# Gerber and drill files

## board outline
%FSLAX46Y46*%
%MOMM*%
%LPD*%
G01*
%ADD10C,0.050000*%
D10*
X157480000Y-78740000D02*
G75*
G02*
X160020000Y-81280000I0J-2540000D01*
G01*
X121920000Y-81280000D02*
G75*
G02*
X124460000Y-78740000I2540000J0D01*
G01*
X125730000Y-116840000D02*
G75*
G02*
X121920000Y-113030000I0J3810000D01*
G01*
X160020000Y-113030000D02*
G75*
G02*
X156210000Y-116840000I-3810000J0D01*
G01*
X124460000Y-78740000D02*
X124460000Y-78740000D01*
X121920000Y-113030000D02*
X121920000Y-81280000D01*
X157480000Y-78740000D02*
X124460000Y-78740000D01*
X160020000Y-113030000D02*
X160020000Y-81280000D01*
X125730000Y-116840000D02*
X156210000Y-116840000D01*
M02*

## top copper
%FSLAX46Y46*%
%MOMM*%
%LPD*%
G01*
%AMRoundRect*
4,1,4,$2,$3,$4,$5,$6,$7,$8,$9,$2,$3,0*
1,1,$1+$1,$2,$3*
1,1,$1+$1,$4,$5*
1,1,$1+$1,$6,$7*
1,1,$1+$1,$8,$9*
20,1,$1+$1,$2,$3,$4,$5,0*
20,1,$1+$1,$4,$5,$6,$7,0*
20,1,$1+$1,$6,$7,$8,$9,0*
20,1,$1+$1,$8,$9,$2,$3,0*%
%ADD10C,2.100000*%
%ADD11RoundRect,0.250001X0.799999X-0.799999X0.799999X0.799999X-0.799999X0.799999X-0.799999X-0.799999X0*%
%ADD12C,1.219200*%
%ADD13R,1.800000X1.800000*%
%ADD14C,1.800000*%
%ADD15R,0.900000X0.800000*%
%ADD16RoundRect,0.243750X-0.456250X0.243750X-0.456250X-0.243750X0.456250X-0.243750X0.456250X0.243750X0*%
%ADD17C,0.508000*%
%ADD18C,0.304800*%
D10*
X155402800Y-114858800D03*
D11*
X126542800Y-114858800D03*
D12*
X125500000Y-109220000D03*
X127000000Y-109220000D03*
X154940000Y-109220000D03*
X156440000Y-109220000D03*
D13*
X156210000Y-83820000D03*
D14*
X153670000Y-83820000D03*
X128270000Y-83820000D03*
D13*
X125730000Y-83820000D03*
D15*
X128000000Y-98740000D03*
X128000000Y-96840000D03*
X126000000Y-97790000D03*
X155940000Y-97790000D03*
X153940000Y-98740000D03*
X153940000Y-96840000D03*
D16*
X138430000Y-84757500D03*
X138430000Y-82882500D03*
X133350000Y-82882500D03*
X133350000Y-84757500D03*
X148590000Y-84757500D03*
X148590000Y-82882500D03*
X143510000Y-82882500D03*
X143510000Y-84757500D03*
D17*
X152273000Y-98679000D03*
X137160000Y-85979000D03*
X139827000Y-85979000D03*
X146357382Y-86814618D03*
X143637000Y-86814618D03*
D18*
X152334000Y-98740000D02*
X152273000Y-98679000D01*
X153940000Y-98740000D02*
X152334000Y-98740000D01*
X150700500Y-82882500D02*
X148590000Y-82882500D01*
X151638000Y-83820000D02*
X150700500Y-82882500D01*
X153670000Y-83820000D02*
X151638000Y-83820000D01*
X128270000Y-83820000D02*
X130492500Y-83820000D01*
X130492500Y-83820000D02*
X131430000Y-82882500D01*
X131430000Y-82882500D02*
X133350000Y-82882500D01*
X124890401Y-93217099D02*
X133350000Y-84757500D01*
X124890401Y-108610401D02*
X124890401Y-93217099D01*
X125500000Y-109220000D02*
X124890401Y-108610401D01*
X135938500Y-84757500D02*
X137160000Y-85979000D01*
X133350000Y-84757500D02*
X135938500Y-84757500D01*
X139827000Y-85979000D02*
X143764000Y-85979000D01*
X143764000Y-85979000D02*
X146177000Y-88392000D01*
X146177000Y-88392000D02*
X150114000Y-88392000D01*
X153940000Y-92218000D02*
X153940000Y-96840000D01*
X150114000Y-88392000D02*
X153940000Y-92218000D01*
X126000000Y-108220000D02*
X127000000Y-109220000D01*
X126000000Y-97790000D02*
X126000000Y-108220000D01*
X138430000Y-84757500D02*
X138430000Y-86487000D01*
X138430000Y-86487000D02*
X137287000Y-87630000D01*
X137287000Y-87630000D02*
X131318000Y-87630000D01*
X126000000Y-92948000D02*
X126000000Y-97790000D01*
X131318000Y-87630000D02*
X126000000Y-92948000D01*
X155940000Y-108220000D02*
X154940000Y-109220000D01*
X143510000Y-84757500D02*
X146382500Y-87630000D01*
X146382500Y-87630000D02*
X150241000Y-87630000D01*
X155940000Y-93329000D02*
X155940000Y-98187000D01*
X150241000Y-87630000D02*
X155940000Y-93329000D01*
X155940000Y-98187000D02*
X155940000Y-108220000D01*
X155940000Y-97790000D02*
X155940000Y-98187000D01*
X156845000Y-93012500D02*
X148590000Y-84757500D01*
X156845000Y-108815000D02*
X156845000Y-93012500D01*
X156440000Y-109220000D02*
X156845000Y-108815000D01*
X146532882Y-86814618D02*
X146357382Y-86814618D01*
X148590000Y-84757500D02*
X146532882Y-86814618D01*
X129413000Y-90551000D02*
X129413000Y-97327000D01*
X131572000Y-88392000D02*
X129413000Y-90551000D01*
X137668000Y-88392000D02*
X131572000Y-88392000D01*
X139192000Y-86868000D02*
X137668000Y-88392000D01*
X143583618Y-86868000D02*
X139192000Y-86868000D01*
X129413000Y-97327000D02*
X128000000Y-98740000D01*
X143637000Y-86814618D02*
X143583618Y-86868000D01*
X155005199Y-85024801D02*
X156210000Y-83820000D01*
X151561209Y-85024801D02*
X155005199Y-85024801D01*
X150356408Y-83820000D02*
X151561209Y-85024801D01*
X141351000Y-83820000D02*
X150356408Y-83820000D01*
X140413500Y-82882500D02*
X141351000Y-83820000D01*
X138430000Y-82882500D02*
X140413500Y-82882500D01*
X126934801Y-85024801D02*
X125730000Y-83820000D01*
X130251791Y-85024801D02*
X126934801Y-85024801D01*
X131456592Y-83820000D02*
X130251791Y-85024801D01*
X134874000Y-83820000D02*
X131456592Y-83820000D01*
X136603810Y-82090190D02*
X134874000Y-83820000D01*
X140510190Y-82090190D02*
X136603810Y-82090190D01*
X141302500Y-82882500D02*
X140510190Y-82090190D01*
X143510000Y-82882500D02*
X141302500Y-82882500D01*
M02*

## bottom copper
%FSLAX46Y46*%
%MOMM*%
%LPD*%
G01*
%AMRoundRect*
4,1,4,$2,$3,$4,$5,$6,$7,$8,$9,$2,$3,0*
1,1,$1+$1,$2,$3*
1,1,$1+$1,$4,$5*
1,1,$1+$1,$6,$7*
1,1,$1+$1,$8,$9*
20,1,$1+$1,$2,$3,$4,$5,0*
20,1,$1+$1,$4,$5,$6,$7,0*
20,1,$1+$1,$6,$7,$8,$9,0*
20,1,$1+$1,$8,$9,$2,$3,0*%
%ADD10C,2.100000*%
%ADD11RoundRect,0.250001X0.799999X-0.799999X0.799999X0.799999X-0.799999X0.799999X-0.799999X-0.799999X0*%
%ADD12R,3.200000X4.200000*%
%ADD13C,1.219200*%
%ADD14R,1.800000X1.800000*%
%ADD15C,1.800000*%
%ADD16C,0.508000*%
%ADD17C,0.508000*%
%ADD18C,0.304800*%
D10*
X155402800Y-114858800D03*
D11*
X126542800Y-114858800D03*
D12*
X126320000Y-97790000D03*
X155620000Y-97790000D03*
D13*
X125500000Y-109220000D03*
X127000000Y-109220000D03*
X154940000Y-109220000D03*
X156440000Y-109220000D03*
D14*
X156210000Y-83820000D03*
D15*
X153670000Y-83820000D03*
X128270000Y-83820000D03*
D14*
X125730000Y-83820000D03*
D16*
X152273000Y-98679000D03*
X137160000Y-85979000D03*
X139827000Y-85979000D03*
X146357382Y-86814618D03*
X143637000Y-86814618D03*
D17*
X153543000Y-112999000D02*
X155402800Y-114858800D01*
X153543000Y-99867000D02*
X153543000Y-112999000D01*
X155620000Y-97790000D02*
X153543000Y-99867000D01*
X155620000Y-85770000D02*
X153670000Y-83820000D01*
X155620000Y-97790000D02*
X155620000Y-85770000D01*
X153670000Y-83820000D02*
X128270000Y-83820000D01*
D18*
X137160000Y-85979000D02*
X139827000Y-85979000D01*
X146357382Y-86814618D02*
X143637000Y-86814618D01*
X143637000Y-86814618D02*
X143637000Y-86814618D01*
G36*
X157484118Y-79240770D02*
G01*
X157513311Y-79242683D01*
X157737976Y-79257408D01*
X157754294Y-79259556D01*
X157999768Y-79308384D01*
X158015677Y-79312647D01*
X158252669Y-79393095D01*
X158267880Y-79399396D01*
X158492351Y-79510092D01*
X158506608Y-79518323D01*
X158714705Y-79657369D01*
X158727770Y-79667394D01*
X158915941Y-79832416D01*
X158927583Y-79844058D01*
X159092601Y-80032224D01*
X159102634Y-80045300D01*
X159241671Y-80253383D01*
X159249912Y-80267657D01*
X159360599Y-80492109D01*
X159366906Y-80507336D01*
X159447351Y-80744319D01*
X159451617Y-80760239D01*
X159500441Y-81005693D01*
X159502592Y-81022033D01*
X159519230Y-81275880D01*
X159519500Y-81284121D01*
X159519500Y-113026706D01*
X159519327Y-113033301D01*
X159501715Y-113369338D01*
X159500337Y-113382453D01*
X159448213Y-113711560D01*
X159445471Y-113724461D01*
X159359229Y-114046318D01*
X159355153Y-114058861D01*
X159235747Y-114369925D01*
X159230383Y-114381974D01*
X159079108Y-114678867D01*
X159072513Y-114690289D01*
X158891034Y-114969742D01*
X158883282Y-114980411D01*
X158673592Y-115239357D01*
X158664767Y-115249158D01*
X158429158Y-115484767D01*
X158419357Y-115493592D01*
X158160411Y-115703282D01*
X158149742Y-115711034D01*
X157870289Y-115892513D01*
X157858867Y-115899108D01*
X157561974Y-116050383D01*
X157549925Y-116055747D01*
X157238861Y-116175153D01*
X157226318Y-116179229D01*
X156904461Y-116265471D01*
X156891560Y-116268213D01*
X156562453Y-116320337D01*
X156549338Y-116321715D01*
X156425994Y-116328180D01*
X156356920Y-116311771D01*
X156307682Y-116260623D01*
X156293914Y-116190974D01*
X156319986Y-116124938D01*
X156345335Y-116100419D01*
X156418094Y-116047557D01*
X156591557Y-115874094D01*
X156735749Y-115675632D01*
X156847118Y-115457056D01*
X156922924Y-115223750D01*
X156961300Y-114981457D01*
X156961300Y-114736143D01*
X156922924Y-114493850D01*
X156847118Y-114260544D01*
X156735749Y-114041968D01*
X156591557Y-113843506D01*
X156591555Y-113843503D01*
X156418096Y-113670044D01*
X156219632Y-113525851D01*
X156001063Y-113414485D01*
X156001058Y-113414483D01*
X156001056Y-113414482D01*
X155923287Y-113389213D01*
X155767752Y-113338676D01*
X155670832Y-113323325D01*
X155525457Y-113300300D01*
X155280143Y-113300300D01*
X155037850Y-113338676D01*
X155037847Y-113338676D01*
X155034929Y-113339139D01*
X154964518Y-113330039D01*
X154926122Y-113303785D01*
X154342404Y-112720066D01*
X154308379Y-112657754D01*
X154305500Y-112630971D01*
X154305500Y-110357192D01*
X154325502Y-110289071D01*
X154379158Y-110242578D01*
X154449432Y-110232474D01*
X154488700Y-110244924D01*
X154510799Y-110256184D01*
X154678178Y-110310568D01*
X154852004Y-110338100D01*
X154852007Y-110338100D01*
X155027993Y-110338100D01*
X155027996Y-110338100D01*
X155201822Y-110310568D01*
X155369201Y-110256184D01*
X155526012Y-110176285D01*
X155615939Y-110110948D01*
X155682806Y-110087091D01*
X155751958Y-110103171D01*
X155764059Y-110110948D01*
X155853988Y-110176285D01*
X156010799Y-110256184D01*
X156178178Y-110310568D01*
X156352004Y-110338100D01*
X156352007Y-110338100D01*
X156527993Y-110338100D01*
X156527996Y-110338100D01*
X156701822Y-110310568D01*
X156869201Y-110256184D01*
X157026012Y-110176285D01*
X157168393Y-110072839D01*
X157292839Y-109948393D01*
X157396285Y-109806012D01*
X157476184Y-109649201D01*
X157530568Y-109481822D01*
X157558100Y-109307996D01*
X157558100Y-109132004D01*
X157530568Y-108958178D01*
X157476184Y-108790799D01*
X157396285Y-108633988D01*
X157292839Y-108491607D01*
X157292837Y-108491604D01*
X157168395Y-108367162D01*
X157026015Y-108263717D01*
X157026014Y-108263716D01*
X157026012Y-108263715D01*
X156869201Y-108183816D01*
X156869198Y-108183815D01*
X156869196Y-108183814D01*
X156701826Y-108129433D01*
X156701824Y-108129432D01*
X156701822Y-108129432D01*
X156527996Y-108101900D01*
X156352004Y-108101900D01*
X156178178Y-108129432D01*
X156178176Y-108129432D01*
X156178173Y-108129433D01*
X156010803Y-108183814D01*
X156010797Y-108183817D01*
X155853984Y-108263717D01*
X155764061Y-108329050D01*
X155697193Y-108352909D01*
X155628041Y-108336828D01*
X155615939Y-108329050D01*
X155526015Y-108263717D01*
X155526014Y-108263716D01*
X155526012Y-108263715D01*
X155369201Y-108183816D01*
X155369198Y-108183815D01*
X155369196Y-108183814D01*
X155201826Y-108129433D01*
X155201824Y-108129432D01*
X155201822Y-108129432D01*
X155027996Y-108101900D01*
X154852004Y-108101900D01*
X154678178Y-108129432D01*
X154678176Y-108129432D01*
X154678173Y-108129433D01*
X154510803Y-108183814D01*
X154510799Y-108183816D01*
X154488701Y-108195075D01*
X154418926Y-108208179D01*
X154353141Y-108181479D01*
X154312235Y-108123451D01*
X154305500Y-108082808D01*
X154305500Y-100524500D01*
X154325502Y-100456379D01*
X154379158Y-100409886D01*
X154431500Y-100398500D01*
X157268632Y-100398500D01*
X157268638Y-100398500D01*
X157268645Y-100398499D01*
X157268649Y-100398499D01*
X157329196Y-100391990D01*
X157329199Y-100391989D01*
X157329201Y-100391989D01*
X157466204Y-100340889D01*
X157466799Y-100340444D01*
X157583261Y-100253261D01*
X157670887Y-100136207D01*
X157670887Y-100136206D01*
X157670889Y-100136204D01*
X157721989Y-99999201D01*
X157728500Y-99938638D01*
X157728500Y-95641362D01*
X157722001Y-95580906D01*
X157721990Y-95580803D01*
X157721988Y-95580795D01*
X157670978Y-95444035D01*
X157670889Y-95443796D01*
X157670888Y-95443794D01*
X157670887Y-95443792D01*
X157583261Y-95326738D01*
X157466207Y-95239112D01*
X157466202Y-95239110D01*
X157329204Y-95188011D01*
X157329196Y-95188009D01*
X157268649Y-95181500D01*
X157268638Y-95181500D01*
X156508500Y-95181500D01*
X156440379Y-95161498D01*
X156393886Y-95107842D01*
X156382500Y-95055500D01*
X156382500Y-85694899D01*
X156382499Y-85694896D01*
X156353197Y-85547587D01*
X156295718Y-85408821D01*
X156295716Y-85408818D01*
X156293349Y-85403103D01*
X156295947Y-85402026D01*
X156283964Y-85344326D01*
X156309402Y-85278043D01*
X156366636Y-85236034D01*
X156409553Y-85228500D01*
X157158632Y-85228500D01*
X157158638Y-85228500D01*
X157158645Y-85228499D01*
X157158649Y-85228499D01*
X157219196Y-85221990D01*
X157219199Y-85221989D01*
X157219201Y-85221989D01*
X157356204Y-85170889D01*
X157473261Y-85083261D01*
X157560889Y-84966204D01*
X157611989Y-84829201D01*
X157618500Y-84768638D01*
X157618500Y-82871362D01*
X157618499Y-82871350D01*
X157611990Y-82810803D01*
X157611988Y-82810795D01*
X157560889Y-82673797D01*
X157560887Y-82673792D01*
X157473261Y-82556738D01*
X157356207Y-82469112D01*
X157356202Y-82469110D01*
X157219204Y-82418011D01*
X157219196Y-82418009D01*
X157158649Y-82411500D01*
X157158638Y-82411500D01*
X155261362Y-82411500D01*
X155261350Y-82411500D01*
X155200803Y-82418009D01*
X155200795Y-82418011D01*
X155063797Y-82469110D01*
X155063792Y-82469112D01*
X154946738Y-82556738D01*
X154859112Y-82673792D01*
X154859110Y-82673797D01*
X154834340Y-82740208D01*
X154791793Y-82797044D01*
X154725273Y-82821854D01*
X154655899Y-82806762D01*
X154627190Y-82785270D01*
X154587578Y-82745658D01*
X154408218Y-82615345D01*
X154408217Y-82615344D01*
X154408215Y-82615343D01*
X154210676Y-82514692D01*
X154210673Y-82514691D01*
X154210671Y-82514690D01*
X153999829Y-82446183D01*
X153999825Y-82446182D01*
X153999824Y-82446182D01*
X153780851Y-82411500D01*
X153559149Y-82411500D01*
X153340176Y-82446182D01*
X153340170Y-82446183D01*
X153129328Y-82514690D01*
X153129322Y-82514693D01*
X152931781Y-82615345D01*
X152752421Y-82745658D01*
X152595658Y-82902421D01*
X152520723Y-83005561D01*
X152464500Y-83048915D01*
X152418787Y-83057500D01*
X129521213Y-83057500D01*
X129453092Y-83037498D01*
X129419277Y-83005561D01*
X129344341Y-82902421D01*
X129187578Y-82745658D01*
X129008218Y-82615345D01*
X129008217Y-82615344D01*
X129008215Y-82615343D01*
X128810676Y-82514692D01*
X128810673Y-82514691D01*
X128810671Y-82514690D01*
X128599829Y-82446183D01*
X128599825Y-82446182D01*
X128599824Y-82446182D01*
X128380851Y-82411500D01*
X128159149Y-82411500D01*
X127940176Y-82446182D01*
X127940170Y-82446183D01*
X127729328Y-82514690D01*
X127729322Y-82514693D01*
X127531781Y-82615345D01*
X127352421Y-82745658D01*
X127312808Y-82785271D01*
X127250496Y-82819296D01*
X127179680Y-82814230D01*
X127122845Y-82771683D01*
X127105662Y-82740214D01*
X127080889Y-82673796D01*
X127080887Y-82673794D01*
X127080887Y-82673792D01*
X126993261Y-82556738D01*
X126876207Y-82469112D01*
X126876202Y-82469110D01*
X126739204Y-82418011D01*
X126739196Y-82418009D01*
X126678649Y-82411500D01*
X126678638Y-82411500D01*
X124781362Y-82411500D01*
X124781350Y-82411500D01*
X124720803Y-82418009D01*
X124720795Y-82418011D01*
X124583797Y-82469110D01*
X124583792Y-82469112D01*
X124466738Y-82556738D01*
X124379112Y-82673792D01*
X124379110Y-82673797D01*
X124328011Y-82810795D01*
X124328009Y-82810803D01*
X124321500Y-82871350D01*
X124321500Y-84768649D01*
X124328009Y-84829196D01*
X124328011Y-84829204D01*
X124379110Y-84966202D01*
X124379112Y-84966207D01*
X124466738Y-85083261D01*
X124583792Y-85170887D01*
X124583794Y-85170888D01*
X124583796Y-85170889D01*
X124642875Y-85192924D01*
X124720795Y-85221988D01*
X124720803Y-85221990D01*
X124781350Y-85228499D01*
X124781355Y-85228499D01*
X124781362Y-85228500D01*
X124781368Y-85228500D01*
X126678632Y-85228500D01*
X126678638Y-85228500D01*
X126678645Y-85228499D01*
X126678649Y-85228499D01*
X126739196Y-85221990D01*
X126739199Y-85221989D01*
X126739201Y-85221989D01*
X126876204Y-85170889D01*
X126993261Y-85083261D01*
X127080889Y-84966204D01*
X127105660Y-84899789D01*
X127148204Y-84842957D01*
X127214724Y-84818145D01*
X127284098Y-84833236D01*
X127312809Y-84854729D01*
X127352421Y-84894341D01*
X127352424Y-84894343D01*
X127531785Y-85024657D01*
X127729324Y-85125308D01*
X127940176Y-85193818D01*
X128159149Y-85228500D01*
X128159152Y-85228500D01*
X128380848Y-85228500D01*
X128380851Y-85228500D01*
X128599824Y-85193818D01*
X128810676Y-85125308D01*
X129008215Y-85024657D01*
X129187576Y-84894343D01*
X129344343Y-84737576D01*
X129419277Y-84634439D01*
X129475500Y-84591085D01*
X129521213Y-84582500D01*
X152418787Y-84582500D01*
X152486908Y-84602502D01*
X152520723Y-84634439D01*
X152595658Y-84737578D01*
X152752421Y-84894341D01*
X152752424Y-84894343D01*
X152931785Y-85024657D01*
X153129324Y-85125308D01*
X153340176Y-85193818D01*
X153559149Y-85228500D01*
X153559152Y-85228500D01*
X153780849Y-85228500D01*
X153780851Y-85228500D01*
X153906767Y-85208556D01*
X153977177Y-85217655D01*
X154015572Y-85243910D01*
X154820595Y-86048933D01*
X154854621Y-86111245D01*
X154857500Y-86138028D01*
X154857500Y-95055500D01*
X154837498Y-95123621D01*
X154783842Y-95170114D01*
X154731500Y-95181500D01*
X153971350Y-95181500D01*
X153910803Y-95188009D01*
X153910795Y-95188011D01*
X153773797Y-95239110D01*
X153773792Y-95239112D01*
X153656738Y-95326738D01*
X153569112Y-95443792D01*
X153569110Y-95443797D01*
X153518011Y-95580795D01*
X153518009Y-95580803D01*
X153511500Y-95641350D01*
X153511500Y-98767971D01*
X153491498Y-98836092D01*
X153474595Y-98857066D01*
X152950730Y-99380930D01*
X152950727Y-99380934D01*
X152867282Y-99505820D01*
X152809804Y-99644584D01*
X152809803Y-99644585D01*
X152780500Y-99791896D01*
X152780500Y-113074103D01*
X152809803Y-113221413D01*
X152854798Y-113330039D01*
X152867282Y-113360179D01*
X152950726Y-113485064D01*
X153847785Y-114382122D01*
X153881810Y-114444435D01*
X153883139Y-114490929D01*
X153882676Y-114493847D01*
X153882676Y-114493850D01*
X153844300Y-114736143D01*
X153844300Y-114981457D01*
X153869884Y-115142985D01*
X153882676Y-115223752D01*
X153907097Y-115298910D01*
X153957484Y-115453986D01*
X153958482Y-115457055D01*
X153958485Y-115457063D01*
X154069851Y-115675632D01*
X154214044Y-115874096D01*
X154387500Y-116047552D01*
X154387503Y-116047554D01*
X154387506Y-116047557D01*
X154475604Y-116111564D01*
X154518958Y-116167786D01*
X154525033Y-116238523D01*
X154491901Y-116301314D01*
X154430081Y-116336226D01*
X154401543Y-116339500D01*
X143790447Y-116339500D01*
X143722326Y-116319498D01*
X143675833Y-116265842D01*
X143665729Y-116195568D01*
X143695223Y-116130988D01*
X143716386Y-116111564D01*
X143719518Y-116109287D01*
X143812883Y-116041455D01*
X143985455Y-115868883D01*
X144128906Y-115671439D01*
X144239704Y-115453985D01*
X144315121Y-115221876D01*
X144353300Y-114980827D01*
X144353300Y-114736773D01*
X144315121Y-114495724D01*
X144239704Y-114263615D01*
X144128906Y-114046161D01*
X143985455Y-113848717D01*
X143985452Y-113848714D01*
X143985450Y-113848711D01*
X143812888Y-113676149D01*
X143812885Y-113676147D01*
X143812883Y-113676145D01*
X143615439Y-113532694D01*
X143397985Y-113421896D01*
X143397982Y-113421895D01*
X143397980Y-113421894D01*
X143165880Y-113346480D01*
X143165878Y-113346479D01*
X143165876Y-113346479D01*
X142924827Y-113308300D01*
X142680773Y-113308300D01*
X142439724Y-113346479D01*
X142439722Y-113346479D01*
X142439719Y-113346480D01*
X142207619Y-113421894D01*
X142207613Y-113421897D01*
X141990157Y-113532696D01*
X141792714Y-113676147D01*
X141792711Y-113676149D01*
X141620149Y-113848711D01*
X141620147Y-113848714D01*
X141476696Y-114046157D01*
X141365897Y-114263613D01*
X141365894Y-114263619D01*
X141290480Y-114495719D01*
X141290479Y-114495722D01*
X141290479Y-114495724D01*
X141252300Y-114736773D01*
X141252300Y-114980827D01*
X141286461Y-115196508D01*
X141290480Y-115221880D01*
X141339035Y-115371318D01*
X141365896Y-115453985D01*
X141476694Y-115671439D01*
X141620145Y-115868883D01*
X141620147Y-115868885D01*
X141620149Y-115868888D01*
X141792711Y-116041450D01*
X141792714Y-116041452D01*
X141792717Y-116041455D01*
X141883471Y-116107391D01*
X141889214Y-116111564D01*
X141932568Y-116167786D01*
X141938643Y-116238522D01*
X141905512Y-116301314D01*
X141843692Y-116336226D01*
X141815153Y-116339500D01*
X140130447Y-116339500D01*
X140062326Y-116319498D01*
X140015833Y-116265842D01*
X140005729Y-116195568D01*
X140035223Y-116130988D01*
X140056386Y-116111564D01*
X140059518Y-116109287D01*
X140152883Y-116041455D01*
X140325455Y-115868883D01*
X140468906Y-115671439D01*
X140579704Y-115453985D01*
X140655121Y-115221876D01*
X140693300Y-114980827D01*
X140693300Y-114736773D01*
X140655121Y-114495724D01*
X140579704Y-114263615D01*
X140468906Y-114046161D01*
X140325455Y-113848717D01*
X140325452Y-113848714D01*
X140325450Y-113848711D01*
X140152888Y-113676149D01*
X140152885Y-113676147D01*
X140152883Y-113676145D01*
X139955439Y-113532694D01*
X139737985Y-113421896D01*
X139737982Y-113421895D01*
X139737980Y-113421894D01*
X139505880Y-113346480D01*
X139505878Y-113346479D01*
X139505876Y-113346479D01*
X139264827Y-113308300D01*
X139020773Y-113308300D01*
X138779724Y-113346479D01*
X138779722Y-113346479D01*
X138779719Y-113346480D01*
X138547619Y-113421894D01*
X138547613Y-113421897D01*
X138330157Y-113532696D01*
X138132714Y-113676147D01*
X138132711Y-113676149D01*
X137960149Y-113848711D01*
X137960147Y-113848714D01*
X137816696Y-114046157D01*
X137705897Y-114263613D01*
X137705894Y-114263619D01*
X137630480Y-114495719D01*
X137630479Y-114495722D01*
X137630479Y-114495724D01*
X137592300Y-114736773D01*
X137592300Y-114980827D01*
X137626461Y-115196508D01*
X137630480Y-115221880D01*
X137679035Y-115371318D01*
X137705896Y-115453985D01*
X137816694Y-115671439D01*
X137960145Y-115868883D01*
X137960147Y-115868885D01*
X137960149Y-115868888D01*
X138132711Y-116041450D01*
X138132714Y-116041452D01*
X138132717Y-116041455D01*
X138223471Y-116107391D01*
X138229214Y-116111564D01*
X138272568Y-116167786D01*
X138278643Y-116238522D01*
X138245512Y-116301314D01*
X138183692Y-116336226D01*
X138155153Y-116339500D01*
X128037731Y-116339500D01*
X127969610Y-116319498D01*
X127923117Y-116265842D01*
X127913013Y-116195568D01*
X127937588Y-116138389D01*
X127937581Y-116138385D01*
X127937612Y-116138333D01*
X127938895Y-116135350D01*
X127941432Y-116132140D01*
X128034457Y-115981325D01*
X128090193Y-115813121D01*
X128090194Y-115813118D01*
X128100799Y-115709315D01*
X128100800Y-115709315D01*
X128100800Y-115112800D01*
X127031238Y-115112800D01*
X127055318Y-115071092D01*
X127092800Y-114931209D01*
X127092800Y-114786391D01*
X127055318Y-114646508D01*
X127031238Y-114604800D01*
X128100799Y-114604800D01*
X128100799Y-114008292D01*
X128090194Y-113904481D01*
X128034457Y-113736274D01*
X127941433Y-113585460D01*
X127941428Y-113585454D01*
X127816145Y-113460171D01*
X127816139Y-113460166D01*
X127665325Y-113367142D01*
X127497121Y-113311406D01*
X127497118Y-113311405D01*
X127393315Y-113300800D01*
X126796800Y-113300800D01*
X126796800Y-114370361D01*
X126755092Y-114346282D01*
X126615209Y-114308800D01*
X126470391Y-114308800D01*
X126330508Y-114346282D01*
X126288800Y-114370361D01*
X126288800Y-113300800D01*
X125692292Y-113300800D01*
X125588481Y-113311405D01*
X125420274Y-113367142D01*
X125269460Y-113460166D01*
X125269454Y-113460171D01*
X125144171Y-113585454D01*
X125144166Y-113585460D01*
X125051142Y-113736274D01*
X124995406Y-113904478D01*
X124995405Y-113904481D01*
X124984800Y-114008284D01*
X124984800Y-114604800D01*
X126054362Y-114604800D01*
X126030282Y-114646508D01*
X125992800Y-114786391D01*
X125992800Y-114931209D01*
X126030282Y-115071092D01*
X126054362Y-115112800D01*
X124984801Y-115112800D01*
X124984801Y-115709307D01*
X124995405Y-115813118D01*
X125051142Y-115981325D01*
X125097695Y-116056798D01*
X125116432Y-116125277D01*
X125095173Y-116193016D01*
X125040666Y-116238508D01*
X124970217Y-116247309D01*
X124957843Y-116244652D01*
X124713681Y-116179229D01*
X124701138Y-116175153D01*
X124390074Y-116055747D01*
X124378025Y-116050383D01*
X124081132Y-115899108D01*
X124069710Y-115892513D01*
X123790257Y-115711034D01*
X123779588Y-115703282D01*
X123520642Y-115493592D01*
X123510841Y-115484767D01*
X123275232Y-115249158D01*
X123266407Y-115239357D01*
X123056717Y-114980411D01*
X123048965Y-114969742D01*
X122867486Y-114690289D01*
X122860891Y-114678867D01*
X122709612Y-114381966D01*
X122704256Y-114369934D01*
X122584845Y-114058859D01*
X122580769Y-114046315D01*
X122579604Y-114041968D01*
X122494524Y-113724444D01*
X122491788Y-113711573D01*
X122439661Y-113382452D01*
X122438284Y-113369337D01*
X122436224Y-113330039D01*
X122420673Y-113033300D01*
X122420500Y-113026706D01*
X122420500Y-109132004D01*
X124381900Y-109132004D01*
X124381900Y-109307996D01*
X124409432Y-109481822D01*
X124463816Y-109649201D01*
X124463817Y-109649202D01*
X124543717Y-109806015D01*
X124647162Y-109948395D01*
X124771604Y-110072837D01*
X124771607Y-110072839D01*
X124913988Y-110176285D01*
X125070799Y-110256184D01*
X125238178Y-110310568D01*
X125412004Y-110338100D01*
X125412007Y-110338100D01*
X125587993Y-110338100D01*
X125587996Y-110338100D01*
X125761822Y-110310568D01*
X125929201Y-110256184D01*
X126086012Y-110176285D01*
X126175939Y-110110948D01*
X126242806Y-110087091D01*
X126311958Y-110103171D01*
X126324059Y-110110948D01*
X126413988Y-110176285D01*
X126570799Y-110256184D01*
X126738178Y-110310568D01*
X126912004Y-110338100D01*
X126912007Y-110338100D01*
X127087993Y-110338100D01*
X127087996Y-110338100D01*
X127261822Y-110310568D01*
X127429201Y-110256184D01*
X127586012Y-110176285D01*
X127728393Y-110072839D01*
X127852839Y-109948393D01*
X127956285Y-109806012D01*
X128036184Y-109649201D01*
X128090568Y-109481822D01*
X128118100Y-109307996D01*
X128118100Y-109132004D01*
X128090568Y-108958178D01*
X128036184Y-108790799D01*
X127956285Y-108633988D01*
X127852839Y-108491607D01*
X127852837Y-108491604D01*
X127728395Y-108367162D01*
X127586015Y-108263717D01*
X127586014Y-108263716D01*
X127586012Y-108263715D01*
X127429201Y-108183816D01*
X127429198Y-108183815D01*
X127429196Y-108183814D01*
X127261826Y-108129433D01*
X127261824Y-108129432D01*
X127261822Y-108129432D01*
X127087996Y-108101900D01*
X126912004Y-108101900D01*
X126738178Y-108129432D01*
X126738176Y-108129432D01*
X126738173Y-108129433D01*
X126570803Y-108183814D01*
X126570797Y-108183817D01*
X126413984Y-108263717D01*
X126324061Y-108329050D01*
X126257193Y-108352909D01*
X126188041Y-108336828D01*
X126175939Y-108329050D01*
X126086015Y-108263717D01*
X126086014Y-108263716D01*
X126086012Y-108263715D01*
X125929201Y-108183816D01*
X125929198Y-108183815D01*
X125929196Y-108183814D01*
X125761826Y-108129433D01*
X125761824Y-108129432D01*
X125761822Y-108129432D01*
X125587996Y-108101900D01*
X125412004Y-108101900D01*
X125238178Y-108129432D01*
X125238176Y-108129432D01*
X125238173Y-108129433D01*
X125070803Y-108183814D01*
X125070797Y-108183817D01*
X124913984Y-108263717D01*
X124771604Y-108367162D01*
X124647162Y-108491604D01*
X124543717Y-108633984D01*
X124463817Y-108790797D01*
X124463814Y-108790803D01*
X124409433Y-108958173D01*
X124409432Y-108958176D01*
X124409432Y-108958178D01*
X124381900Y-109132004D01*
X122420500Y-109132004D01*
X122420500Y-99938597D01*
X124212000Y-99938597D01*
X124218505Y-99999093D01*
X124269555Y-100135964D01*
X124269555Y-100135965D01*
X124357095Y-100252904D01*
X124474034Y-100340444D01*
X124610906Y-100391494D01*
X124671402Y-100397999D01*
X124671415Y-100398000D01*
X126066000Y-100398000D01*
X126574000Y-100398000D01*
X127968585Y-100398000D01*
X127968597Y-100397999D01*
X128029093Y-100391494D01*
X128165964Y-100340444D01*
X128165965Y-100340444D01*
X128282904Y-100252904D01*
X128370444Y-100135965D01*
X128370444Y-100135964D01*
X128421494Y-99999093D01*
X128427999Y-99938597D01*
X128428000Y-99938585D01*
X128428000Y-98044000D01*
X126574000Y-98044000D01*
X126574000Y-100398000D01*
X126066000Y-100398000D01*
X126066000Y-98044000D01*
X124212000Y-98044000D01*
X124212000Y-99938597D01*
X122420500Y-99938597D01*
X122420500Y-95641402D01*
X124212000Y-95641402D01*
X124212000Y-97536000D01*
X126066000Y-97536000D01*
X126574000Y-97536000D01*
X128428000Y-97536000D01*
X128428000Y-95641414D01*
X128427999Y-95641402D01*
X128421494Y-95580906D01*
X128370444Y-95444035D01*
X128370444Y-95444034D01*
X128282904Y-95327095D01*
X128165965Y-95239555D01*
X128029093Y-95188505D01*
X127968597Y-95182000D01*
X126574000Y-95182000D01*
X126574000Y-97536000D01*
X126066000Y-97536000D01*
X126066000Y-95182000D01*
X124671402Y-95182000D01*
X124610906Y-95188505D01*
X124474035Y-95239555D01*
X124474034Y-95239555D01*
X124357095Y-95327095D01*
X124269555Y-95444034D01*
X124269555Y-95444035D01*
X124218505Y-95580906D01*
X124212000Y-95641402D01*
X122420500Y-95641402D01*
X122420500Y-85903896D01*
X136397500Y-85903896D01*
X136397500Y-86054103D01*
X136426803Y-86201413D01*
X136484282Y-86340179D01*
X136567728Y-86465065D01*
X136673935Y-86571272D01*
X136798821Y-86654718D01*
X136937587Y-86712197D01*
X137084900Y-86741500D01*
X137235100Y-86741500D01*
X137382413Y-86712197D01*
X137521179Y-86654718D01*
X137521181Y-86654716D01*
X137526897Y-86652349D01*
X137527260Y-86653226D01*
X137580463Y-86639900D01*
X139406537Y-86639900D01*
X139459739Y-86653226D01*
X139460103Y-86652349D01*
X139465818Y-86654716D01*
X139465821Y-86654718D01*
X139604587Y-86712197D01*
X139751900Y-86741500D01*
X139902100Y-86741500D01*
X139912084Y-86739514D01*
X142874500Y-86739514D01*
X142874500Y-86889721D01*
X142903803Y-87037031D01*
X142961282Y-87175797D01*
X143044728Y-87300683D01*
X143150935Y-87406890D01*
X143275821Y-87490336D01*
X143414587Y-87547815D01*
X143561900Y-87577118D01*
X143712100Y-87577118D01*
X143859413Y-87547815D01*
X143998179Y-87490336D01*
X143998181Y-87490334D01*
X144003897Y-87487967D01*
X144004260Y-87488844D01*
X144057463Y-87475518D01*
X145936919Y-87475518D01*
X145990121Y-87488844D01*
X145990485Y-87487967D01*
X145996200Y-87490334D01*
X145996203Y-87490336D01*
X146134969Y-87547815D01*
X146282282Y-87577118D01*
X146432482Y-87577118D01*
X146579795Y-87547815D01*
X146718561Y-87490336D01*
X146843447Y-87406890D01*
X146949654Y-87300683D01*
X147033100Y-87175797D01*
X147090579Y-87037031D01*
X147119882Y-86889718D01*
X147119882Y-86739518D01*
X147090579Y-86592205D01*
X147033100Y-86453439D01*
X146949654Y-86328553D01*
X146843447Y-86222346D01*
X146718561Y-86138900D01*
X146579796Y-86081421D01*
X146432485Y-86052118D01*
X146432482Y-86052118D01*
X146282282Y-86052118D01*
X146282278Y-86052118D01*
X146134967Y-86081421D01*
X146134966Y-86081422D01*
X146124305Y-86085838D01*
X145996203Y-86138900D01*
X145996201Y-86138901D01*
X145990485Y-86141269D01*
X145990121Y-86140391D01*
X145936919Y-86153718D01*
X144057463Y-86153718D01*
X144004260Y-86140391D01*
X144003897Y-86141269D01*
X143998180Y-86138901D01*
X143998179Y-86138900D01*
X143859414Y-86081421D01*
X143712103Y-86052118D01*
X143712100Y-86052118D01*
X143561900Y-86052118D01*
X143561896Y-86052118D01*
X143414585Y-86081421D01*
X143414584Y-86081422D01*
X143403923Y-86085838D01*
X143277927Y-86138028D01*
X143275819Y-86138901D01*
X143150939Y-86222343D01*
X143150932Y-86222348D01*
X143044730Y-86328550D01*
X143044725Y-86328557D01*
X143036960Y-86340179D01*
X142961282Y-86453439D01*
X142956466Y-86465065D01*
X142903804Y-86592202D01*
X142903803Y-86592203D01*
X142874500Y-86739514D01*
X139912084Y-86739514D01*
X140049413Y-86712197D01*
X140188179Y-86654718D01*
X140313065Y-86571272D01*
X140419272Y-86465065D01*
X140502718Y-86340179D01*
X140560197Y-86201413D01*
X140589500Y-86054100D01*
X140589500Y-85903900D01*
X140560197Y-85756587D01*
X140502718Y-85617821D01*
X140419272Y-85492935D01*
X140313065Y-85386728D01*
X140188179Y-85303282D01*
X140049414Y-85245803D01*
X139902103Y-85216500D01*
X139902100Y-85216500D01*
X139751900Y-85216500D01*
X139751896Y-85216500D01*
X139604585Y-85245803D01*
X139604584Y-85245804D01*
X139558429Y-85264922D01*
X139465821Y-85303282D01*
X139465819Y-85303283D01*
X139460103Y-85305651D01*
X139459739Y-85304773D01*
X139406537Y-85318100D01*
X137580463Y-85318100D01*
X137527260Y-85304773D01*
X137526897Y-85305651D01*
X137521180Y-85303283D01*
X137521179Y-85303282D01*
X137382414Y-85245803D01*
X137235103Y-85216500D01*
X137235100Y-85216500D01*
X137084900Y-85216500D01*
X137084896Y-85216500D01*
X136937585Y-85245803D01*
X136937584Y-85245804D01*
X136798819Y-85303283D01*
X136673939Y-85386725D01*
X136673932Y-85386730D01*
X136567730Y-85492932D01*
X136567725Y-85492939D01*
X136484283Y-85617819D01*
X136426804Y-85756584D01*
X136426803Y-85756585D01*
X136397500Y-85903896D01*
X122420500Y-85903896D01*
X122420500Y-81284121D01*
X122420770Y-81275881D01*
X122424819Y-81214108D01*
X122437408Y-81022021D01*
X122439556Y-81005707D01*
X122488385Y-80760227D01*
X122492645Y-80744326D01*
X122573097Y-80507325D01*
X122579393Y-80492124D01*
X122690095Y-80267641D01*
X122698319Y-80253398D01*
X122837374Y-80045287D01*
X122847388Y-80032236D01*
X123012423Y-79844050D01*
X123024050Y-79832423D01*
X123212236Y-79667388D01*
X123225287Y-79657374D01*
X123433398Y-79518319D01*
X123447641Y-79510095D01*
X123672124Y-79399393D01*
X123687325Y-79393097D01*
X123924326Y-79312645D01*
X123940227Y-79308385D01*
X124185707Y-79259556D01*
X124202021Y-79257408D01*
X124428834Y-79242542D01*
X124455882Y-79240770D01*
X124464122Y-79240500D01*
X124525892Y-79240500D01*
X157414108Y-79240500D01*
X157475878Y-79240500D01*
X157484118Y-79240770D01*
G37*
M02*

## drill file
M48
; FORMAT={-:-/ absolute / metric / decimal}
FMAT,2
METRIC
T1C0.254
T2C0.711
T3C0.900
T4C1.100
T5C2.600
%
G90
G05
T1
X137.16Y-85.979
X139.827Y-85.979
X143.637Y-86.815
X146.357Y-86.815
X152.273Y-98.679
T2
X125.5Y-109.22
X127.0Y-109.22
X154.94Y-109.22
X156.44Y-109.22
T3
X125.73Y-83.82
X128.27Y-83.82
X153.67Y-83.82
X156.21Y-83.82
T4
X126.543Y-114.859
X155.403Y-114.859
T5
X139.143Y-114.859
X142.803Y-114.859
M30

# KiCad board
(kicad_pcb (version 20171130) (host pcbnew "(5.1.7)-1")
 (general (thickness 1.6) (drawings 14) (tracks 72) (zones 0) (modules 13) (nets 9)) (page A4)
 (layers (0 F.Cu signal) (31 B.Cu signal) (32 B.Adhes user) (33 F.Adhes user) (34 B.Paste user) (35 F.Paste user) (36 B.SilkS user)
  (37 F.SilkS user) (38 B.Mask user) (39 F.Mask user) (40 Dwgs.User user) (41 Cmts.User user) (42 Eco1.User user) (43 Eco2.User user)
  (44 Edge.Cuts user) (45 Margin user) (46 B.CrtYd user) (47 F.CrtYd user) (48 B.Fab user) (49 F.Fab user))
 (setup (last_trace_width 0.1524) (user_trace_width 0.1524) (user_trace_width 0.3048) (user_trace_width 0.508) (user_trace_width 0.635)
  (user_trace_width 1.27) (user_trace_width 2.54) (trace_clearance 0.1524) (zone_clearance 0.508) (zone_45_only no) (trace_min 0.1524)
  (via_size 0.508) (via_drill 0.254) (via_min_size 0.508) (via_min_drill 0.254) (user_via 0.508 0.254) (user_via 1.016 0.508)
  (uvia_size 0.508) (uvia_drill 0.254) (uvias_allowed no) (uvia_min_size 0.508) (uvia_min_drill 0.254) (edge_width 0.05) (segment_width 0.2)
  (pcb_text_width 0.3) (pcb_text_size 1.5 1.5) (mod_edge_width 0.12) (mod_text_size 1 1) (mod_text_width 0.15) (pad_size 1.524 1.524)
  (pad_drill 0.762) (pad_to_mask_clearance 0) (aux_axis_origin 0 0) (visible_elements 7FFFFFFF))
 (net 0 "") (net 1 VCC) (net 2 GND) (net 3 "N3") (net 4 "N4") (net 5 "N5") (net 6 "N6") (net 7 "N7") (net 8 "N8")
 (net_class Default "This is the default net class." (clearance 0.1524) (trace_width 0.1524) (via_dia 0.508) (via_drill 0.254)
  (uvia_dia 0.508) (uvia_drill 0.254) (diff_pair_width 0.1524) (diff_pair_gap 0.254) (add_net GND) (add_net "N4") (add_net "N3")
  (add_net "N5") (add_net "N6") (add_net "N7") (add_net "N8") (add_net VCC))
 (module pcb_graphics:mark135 (layer F.Cu) (at 140.97 99.06)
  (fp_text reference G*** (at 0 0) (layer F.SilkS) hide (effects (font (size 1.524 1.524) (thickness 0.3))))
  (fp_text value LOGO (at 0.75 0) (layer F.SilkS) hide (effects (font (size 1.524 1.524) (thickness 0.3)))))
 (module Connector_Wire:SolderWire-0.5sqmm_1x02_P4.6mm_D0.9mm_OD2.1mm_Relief (layer F.Cu) (at 140.5128 114.8588)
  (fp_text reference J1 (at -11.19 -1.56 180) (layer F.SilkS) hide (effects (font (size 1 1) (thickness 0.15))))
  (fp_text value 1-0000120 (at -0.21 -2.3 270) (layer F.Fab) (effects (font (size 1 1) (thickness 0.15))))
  (pad "" np_thru_hole circle (at 2.29 0 270) (size 2.6 2.6) (drill 2.6) (layers *.Cu *.Mask))
  (pad "" np_thru_hole circle (at -1.37 0 90) (size 2.6 2.6) (drill 2.6) (layers *.Cu *.Mask))
  (pad 2 thru_hole circle (at 14.89 0 270) (size 2.1 2.1) (drill 1.1) (layers *.Cu *.Mask) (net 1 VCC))
  (pad 1 thru_hole roundrect (at -13.97 0 90) (size 2.1 2.1) (drill 1.1) (layers *.Cu *.Mask) (roundrect_rratio 0.119048) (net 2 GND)))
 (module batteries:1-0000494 (layer B.Cu) (at 140.97 97.79 180)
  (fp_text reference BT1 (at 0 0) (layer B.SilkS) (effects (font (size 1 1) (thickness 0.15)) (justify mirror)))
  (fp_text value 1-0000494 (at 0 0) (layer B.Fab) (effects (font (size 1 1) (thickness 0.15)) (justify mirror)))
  (pad 2 smd rect (at 14.65 0 180) (size 3.2 4.2) (layers B.Cu B.Paste B.Mask) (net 2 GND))
  (pad 1 smd rect (at -14.65 0 180) (size 3.2 4.2) (layers B.Cu B.Paste B.Mask) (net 1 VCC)))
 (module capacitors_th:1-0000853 (layer F.Cu) (at 127 109.22 180)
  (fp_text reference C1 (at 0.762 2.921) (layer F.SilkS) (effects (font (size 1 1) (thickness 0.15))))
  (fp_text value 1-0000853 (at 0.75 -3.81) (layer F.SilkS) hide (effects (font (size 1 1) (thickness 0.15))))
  (pad 2 thru_hole circle (at 1.5 0 180) (size 1.2192 1.2192) (drill 0.7112) (layers *.Cu *.Mask) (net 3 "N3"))
  (pad 1 thru_hole circle (at 0 0 180) (size 1.2192 1.2192) (drill 0.7112) (layers *.Cu *.Mask) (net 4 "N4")))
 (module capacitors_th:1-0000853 (layer F.Cu) (at 154.94 109.22)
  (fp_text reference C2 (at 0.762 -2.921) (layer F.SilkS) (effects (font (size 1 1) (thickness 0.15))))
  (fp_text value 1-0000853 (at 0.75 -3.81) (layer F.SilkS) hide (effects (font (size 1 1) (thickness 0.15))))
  (pad 1 thru_hole circle (at 0 0) (size 1.2192 1.2192) (drill 0.7112) (layers *.Cu *.Mask) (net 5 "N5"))
  (pad 2 thru_hole circle (at 1.5 0) (size 1.2192 1.2192) (drill 0.7112) (layers *.Cu *.Mask) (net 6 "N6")))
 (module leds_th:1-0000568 (layer F.Cu) (at 156.21 83.82 180)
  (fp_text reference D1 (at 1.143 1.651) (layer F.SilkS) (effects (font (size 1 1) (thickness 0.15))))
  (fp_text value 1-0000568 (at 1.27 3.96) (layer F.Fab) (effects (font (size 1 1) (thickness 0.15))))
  (pad 1 thru_hole rect (at 0 0 180) (size 1.8 1.8) (drill 0.9) (layers *.Cu *.Mask) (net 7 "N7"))
  (pad 2 thru_hole circle (at 2.54 0 180) (size 1.8 1.8) (drill 0.9) (layers *.Cu *.Mask) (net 1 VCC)))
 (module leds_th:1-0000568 (layer F.Cu) (at 125.73 83.82)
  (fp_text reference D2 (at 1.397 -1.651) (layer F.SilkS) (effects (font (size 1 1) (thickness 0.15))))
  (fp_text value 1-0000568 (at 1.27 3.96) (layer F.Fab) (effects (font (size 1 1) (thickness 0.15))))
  (pad 2 thru_hole circle (at 2.54 0) (size 1.8 1.8) (drill 0.9) (layers *.Cu *.Mask) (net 1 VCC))
  (pad 1 thru_hole rect (at 0 0) (size 1.8 1.8) (drill 0.9) (layers *.Cu *.Mask) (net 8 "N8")))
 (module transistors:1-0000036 (layer F.Cu) (at 127 97.79 180)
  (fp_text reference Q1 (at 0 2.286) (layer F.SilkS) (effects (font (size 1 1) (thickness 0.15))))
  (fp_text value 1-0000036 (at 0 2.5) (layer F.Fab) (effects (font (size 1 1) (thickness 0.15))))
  (pad 1 smd rect (at -1 -0.95 180) (size 0.9 0.8) (layers F.Cu F.Paste F.Mask) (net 6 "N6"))
  (pad 2 smd rect (at -1 0.95 180) (size 0.9 0.8) (layers F.Cu F.Paste F.Mask) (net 2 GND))
  (pad 3 smd rect (at 1 0 180) (size 0.9 0.8) (layers F.Cu F.Paste F.Mask) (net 4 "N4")))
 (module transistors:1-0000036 (layer F.Cu) (at 154.94 97.79)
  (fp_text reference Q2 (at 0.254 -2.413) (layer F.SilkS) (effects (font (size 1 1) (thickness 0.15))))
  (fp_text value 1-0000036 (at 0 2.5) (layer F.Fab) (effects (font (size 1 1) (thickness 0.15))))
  (pad 3 smd rect (at 1 0) (size 0.9 0.8) (layers F.Cu F.Paste F.Mask) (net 5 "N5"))
  (pad 2 smd rect (at -1 0.95) (size 0.9 0.8) (layers F.Cu F.Paste F.Mask) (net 2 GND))
  (pad 1 smd rect (at -1 -0.95) (size 0.9 0.8) (layers F.Cu F.Paste F.Mask) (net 3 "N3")))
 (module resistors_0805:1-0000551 (layer F.Cu) (at 138.43 83.82 270)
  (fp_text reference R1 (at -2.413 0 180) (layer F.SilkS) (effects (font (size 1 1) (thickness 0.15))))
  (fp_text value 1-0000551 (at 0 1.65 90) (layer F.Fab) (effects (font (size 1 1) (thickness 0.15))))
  (pad 2 smd roundrect (at 0.9375 0 270) (size 0.975 1.4) (layers F.Cu F.Paste F.Mask) (roundrect_rratio 0.25) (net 4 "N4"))
  (pad 1 smd roundrect (at -0.9375 0 270) (size 0.975 1.4) (layers F.Cu F.Paste F.Mask) (roundrect_rratio 0.25) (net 7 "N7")))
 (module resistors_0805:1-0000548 (layer F.Cu) (at 133.35 83.82 270)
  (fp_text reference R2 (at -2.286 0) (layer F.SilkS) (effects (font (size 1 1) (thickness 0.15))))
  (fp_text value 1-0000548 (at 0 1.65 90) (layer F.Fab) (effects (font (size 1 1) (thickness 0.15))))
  (pad 1 smd roundrect (at -0.9375 0 270) (size 0.975 1.4) (layers F.Cu F.Paste F.Mask) (roundrect_rratio 0.25) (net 1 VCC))
  (pad 2 smd roundrect (at 0.9375 0 270) (size 0.975 1.4) (layers F.Cu F.Paste F.Mask) (roundrect_rratio 0.25) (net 3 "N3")))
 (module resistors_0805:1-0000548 (layer F.Cu) (at 148.59 83.82 270)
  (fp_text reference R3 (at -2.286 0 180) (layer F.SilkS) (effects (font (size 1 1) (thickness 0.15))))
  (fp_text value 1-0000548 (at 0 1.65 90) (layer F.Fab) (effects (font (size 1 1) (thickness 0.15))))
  (pad 2 smd roundrect (at 0.9375 0 270) (size 0.975 1.4) (layers F.Cu F.Paste F.Mask) (roundrect_rratio 0.25) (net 6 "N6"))
  (pad 1 smd roundrect (at -0.9375 0 270) (size 0.975 1.4) (layers F.Cu F.Paste F.Mask) (roundrect_rratio 0.25) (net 1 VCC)))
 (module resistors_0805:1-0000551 (layer F.Cu) (at 143.51 83.82 270)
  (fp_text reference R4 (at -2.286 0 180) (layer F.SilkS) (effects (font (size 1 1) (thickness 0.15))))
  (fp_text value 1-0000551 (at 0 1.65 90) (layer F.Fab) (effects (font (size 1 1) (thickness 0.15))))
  (pad 1 smd roundrect (at -0.9375 0 270) (size 0.975 1.4) (layers F.Cu F.Paste F.Mask) (roundrect_rratio 0.25) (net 8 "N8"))
  (pad 2 smd roundrect (at 0.9375 0 270) (size 0.975 1.4) (layers F.Cu F.Paste F.Mask) (roundrect_rratio 0.25) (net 5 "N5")))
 (gr_arc (start 157.48 81.28) (end 160.02 81.28) (angle -90) (layer Edge.Cuts) (width 0.05))
 (gr_arc (start 124.46 81.28) (end 124.46 78.74) (angle -90) (layer Edge.Cuts) (width 0.05))
 (gr_arc (start 125.73 113.03) (end 121.92 113.03) (angle -90) (layer Edge.Cuts) (width 0.05))
 (gr_arc (start 156.21 113.03) (end 156.21 116.84) (angle -90) (layer Edge.Cuts) (width 0.05))
 (gr_line (start 124.46 78.74) (end 124.46 78.74) (layer Edge.Cuts) (width 0.05))
 (gr_line (start 121.92 113.03) (end 121.92 81.28) (layer Edge.Cuts) (width 0.05))
 (gr_line (start 157.48 78.74) (end 124.46 78.74) (layer Edge.Cuts) (width 0.05))
 (gr_line (start 160.02 113.03) (end 160.02 81.28) (layer Edge.Cuts) (width 0.05))
 (gr_line (start 125.73 116.84) (end 156.21 116.84) (layer Edge.Cuts) (width 0.05))
 (via (at 152.273 98.679) (size 0.508) (drill 0.254) (layers F.Cu B.Cu) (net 2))
 (segment (start 152.334 98.74) (end 152.273 98.679) (width 0.3048) (layer F.Cu) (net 2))
 (segment (start 153.94 98.74) (end 152.334 98.74) (width 0.3048) (layer F.Cu) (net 2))
 (segment (start 153.543 112.999) (end 155.4028 114.8588) (width 0.508) (layer B.Cu) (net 1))
 (segment (start 153.543 99.867) (end 153.543 112.999) (width 0.508) (layer B.Cu) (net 1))
 (segment (start 155.62 97.79) (end 153.543 99.867) (width 0.508) (layer B.Cu) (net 1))
 (segment (start 155.62 85.77) (end 153.67 83.82) (width 0.508) (layer B.Cu) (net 1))
 (segment (start 155.62 97.79) (end 155.62 85.77) (width 0.508) (layer B.Cu) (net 1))
 (segment (start 153.67 83.82) (end 128.27 83.82) (width 0.508) (layer B.Cu) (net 1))
 (segment (start 150.7005 82.8825) (end 148.59 82.8825) (width 0.3048) (layer F.Cu) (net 1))
 (segment (start 151.638 83.82) (end 150.7005 82.8825) (width 0.3048) (layer F.Cu) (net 1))
 (segment (start 153.67 83.82) (end 151.638 83.82) (width 0.3048) (layer F.Cu) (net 1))
 (segment (start 128.27 83.82) (end 130.4925 83.82) (width 0.3048) (layer F.Cu) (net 1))
 (segment (start 130.4925 83.82) (end 131.43 82.8825) (width 0.3048) (layer F.Cu) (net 1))
 (segment (start 131.43 82.8825) (end 133.35 82.8825) (width 0.3048) (layer F.Cu) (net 1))
 (segment (start 124.890401 93.217099) (end 133.35 84.7575) (width 0.3048) (layer F.Cu) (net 3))
 (segment (start 124.890401 108.610401) (end 124.890401 93.217099) (width 0.3048) (layer F.Cu) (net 3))
 (segment (start 125.5 109.22) (end 124.890401 108.610401) (width 0.3048) (layer F.Cu) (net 3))
 (via (at 137.16 85.979) (size 0.508) (drill 0.254) (layers F.Cu B.Cu) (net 3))
 (segment (start 135.9385 84.7575) (end 137.16 85.979) (width 0.3048) (layer F.Cu) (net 3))
 (segment (start 133.35 84.7575) (end 135.9385 84.7575) (width 0.3048) (layer F.Cu) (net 3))
 (via (at 139.827 85.979) (size 0.508) (drill 0.254) (layers F.Cu B.Cu) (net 3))
 (segment (start 137.16 85.979) (end 139.827 85.979) (width 0.3048) (layer B.Cu) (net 3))
 (segment (start 139.827 85.979) (end 143.764 85.979) (width 0.3048) (layer F.Cu) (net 3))
 (segment (start 143.764 85.979) (end 146.177 88.392) (width 0.3048) (layer F.Cu) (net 3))
 (segment (start 146.177 88.392) (end 150.114 88.392) (width 0.3048) (layer F.Cu) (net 3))
 (segment (start 153.94 92.218) (end 153.94 96.84) (width 0.3048) (layer F.Cu) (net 3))
 (segment (start 150.114 88.392) (end 153.94 92.218) (width 0.3048) (layer F.Cu) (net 3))
 (segment (start 126 108.22) (end 127 109.22) (width 0.3048) (layer F.Cu) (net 4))
 (segment (start 126 97.79) (end 126 108.22) (width 0.3048) (layer F.Cu) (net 4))
 (segment (start 138.43 84.7575) (end 138.43 86.487) (width 0.3048) (layer F.Cu) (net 4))
 (segment (start 138.43 86.487) (end 137.287 87.63) (width 0.3048) (layer F.Cu) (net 4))
 (segment (start 137.287 87.63) (end 131.318 87.63) (width 0.3048) (layer F.Cu) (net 4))
 (segment (start 126 92.948) (end 126 97.79) (width 0.3048) (layer F.Cu) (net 4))
 (segment (start 131.318 87.63) (end 126 92.948) (width 0.3048) (layer F.Cu) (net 4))
 (segment (start 155.94 108.22) (end 154.94 109.22) (width 0.3048) (layer F.Cu) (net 5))
 (segment (start 143.51 84.7575) (end 146.3825 87.63) (width 0.3048) (layer F.Cu) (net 5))
 (segment (start 146.3825 87.63) (end 150.241 87.63) (width 0.3048) (layer F.Cu) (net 5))
 (segment (start 155.94 93.329) (end 155.94 98.187) (width 0.3048) (layer F.Cu) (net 5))
 (segment (start 150.241 87.63) (end 155.94 93.329) (width 0.3048) (layer F.Cu) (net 5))
 (segment (start 155.94 98.187) (end 155.94 108.22) (width 0.3048) (layer F.Cu) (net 5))
 (segment (start 155.94 97.79) (end 155.94 98.187) (width 0.3048) (layer F.Cu) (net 5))
 (segment (start 156.845 93.0125) (end 148.59 84.7575) (width 0.3048) (layer F.Cu) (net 6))
 (segment (start 156.845 108.815) (end 156.845 93.0125) (width 0.3048) (layer F.Cu) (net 6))
 (segment (start 156.44 109.22) (end 156.845 108.815) (width 0.3048) (layer F.Cu) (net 6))
 (via (at 146.357382 86.814618) (size 0.508) (drill 0.254) (layers F.Cu B.Cu) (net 6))
 (segment (start 146.532882 86.814618) (end 146.357382 86.814618) (width 0.3048) (layer F.Cu) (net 6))
 (segment (start 148.59 84.7575) (end 146.532882 86.814618) (width 0.3048) (layer F.Cu) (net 6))
 (segment (start 146.357382 86.814618) (end 143.637 86.814618) (width 0.3048) (layer B.Cu) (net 6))
 (segment (start 143.637 86.814618) (end 143.637 86.814618) (width 0.3048) (layer B.Cu) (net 6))
 (via (at 143.637 86.814618) (size 0.508) (drill 0.254) (layers F.Cu B.Cu) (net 6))
 (segment (start 129.413 90.551) (end 129.413 97.327) (width 0.3048) (layer F.Cu) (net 6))
 (segment (start 131.572 88.392) (end 129.413 90.551) (width 0.3048) (layer F.Cu) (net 6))
 (segment (start 137.668 88.392) (end 131.572 88.392) (width 0.3048) (layer F.Cu) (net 6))
 (segment (start 139.192 86.868) (end 137.668 88.392) (width 0.3048) (layer F.Cu) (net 6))
 (segment (start 143.583618 86.868) (end 139.192 86.868) (width 0.3048) (layer F.Cu) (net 6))
 (segment (start 129.413 97.327) (end 128 98.74) (width 0.3048) (layer F.Cu) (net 6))
 (segment (start 143.637 86.814618) (end 143.583618 86.868) (width 0.3048) (layer F.Cu) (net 6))
 (segment (start 155.005199 85.024801) (end 156.21 83.82) (width 0.3048) (layer F.Cu) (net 7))
 (segment (start 151.561209 85.024801) (end 155.005199 85.024801) (width 0.3048) (layer F.Cu) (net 7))
 (segment (start 150.356408 83.82) (end 151.561209 85.024801) (width 0.3048) (layer F.Cu) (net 7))
 (segment (start 141.351 83.82) (end 150.356408 83.82) (width 0.3048) (layer F.Cu) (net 7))
 (segment (start 140.4135 82.8825) (end 141.351 83.82) (width 0.3048) (layer F.Cu) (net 7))
 (segment (start 138.43 82.8825) (end 140.4135 82.8825) (width 0.3048) (layer F.Cu) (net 7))
 (segment (start 126.934801 85.024801) (end 125.73 83.82) (width 0.3048) (layer F.Cu) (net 8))
 (segment (start 130.251791 85.024801) (end 126.934801 85.024801) (width 0.3048) (layer F.Cu) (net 8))
 (segment (start 131.456592 83.82) (end 130.251791 85.024801) (width 0.3048) (layer F.Cu) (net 8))
 (segment (start 134.874 83.82) (end 131.456592 83.82) (width 0.3048) (layer F.Cu) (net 8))
 (segment (start 136.60381 82.09019) (end 134.874 83.82) (width 0.3048) (layer F.Cu) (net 8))
 (segment (start 140.51019 82.09019) (end 136.60381 82.09019) (width 0.3048) (layer F.Cu) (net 8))
 (segment (start 141.3025 82.8825) (end 140.51019 82.09019) (width 0.3048) (layer F.Cu) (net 8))
 (segment (start 143.51 82.8825) (end 141.3025 82.8825) (width 0.3048) (layer F.Cu) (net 8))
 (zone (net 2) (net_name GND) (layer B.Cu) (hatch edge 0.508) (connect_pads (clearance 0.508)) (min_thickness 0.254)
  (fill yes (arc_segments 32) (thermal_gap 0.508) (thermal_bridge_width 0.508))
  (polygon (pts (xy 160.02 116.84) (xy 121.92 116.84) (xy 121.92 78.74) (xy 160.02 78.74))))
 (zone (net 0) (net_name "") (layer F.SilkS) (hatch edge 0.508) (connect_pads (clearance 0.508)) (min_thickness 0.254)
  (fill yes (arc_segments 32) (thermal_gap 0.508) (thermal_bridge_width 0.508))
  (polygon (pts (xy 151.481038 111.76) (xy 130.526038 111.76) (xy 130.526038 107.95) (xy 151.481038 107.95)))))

